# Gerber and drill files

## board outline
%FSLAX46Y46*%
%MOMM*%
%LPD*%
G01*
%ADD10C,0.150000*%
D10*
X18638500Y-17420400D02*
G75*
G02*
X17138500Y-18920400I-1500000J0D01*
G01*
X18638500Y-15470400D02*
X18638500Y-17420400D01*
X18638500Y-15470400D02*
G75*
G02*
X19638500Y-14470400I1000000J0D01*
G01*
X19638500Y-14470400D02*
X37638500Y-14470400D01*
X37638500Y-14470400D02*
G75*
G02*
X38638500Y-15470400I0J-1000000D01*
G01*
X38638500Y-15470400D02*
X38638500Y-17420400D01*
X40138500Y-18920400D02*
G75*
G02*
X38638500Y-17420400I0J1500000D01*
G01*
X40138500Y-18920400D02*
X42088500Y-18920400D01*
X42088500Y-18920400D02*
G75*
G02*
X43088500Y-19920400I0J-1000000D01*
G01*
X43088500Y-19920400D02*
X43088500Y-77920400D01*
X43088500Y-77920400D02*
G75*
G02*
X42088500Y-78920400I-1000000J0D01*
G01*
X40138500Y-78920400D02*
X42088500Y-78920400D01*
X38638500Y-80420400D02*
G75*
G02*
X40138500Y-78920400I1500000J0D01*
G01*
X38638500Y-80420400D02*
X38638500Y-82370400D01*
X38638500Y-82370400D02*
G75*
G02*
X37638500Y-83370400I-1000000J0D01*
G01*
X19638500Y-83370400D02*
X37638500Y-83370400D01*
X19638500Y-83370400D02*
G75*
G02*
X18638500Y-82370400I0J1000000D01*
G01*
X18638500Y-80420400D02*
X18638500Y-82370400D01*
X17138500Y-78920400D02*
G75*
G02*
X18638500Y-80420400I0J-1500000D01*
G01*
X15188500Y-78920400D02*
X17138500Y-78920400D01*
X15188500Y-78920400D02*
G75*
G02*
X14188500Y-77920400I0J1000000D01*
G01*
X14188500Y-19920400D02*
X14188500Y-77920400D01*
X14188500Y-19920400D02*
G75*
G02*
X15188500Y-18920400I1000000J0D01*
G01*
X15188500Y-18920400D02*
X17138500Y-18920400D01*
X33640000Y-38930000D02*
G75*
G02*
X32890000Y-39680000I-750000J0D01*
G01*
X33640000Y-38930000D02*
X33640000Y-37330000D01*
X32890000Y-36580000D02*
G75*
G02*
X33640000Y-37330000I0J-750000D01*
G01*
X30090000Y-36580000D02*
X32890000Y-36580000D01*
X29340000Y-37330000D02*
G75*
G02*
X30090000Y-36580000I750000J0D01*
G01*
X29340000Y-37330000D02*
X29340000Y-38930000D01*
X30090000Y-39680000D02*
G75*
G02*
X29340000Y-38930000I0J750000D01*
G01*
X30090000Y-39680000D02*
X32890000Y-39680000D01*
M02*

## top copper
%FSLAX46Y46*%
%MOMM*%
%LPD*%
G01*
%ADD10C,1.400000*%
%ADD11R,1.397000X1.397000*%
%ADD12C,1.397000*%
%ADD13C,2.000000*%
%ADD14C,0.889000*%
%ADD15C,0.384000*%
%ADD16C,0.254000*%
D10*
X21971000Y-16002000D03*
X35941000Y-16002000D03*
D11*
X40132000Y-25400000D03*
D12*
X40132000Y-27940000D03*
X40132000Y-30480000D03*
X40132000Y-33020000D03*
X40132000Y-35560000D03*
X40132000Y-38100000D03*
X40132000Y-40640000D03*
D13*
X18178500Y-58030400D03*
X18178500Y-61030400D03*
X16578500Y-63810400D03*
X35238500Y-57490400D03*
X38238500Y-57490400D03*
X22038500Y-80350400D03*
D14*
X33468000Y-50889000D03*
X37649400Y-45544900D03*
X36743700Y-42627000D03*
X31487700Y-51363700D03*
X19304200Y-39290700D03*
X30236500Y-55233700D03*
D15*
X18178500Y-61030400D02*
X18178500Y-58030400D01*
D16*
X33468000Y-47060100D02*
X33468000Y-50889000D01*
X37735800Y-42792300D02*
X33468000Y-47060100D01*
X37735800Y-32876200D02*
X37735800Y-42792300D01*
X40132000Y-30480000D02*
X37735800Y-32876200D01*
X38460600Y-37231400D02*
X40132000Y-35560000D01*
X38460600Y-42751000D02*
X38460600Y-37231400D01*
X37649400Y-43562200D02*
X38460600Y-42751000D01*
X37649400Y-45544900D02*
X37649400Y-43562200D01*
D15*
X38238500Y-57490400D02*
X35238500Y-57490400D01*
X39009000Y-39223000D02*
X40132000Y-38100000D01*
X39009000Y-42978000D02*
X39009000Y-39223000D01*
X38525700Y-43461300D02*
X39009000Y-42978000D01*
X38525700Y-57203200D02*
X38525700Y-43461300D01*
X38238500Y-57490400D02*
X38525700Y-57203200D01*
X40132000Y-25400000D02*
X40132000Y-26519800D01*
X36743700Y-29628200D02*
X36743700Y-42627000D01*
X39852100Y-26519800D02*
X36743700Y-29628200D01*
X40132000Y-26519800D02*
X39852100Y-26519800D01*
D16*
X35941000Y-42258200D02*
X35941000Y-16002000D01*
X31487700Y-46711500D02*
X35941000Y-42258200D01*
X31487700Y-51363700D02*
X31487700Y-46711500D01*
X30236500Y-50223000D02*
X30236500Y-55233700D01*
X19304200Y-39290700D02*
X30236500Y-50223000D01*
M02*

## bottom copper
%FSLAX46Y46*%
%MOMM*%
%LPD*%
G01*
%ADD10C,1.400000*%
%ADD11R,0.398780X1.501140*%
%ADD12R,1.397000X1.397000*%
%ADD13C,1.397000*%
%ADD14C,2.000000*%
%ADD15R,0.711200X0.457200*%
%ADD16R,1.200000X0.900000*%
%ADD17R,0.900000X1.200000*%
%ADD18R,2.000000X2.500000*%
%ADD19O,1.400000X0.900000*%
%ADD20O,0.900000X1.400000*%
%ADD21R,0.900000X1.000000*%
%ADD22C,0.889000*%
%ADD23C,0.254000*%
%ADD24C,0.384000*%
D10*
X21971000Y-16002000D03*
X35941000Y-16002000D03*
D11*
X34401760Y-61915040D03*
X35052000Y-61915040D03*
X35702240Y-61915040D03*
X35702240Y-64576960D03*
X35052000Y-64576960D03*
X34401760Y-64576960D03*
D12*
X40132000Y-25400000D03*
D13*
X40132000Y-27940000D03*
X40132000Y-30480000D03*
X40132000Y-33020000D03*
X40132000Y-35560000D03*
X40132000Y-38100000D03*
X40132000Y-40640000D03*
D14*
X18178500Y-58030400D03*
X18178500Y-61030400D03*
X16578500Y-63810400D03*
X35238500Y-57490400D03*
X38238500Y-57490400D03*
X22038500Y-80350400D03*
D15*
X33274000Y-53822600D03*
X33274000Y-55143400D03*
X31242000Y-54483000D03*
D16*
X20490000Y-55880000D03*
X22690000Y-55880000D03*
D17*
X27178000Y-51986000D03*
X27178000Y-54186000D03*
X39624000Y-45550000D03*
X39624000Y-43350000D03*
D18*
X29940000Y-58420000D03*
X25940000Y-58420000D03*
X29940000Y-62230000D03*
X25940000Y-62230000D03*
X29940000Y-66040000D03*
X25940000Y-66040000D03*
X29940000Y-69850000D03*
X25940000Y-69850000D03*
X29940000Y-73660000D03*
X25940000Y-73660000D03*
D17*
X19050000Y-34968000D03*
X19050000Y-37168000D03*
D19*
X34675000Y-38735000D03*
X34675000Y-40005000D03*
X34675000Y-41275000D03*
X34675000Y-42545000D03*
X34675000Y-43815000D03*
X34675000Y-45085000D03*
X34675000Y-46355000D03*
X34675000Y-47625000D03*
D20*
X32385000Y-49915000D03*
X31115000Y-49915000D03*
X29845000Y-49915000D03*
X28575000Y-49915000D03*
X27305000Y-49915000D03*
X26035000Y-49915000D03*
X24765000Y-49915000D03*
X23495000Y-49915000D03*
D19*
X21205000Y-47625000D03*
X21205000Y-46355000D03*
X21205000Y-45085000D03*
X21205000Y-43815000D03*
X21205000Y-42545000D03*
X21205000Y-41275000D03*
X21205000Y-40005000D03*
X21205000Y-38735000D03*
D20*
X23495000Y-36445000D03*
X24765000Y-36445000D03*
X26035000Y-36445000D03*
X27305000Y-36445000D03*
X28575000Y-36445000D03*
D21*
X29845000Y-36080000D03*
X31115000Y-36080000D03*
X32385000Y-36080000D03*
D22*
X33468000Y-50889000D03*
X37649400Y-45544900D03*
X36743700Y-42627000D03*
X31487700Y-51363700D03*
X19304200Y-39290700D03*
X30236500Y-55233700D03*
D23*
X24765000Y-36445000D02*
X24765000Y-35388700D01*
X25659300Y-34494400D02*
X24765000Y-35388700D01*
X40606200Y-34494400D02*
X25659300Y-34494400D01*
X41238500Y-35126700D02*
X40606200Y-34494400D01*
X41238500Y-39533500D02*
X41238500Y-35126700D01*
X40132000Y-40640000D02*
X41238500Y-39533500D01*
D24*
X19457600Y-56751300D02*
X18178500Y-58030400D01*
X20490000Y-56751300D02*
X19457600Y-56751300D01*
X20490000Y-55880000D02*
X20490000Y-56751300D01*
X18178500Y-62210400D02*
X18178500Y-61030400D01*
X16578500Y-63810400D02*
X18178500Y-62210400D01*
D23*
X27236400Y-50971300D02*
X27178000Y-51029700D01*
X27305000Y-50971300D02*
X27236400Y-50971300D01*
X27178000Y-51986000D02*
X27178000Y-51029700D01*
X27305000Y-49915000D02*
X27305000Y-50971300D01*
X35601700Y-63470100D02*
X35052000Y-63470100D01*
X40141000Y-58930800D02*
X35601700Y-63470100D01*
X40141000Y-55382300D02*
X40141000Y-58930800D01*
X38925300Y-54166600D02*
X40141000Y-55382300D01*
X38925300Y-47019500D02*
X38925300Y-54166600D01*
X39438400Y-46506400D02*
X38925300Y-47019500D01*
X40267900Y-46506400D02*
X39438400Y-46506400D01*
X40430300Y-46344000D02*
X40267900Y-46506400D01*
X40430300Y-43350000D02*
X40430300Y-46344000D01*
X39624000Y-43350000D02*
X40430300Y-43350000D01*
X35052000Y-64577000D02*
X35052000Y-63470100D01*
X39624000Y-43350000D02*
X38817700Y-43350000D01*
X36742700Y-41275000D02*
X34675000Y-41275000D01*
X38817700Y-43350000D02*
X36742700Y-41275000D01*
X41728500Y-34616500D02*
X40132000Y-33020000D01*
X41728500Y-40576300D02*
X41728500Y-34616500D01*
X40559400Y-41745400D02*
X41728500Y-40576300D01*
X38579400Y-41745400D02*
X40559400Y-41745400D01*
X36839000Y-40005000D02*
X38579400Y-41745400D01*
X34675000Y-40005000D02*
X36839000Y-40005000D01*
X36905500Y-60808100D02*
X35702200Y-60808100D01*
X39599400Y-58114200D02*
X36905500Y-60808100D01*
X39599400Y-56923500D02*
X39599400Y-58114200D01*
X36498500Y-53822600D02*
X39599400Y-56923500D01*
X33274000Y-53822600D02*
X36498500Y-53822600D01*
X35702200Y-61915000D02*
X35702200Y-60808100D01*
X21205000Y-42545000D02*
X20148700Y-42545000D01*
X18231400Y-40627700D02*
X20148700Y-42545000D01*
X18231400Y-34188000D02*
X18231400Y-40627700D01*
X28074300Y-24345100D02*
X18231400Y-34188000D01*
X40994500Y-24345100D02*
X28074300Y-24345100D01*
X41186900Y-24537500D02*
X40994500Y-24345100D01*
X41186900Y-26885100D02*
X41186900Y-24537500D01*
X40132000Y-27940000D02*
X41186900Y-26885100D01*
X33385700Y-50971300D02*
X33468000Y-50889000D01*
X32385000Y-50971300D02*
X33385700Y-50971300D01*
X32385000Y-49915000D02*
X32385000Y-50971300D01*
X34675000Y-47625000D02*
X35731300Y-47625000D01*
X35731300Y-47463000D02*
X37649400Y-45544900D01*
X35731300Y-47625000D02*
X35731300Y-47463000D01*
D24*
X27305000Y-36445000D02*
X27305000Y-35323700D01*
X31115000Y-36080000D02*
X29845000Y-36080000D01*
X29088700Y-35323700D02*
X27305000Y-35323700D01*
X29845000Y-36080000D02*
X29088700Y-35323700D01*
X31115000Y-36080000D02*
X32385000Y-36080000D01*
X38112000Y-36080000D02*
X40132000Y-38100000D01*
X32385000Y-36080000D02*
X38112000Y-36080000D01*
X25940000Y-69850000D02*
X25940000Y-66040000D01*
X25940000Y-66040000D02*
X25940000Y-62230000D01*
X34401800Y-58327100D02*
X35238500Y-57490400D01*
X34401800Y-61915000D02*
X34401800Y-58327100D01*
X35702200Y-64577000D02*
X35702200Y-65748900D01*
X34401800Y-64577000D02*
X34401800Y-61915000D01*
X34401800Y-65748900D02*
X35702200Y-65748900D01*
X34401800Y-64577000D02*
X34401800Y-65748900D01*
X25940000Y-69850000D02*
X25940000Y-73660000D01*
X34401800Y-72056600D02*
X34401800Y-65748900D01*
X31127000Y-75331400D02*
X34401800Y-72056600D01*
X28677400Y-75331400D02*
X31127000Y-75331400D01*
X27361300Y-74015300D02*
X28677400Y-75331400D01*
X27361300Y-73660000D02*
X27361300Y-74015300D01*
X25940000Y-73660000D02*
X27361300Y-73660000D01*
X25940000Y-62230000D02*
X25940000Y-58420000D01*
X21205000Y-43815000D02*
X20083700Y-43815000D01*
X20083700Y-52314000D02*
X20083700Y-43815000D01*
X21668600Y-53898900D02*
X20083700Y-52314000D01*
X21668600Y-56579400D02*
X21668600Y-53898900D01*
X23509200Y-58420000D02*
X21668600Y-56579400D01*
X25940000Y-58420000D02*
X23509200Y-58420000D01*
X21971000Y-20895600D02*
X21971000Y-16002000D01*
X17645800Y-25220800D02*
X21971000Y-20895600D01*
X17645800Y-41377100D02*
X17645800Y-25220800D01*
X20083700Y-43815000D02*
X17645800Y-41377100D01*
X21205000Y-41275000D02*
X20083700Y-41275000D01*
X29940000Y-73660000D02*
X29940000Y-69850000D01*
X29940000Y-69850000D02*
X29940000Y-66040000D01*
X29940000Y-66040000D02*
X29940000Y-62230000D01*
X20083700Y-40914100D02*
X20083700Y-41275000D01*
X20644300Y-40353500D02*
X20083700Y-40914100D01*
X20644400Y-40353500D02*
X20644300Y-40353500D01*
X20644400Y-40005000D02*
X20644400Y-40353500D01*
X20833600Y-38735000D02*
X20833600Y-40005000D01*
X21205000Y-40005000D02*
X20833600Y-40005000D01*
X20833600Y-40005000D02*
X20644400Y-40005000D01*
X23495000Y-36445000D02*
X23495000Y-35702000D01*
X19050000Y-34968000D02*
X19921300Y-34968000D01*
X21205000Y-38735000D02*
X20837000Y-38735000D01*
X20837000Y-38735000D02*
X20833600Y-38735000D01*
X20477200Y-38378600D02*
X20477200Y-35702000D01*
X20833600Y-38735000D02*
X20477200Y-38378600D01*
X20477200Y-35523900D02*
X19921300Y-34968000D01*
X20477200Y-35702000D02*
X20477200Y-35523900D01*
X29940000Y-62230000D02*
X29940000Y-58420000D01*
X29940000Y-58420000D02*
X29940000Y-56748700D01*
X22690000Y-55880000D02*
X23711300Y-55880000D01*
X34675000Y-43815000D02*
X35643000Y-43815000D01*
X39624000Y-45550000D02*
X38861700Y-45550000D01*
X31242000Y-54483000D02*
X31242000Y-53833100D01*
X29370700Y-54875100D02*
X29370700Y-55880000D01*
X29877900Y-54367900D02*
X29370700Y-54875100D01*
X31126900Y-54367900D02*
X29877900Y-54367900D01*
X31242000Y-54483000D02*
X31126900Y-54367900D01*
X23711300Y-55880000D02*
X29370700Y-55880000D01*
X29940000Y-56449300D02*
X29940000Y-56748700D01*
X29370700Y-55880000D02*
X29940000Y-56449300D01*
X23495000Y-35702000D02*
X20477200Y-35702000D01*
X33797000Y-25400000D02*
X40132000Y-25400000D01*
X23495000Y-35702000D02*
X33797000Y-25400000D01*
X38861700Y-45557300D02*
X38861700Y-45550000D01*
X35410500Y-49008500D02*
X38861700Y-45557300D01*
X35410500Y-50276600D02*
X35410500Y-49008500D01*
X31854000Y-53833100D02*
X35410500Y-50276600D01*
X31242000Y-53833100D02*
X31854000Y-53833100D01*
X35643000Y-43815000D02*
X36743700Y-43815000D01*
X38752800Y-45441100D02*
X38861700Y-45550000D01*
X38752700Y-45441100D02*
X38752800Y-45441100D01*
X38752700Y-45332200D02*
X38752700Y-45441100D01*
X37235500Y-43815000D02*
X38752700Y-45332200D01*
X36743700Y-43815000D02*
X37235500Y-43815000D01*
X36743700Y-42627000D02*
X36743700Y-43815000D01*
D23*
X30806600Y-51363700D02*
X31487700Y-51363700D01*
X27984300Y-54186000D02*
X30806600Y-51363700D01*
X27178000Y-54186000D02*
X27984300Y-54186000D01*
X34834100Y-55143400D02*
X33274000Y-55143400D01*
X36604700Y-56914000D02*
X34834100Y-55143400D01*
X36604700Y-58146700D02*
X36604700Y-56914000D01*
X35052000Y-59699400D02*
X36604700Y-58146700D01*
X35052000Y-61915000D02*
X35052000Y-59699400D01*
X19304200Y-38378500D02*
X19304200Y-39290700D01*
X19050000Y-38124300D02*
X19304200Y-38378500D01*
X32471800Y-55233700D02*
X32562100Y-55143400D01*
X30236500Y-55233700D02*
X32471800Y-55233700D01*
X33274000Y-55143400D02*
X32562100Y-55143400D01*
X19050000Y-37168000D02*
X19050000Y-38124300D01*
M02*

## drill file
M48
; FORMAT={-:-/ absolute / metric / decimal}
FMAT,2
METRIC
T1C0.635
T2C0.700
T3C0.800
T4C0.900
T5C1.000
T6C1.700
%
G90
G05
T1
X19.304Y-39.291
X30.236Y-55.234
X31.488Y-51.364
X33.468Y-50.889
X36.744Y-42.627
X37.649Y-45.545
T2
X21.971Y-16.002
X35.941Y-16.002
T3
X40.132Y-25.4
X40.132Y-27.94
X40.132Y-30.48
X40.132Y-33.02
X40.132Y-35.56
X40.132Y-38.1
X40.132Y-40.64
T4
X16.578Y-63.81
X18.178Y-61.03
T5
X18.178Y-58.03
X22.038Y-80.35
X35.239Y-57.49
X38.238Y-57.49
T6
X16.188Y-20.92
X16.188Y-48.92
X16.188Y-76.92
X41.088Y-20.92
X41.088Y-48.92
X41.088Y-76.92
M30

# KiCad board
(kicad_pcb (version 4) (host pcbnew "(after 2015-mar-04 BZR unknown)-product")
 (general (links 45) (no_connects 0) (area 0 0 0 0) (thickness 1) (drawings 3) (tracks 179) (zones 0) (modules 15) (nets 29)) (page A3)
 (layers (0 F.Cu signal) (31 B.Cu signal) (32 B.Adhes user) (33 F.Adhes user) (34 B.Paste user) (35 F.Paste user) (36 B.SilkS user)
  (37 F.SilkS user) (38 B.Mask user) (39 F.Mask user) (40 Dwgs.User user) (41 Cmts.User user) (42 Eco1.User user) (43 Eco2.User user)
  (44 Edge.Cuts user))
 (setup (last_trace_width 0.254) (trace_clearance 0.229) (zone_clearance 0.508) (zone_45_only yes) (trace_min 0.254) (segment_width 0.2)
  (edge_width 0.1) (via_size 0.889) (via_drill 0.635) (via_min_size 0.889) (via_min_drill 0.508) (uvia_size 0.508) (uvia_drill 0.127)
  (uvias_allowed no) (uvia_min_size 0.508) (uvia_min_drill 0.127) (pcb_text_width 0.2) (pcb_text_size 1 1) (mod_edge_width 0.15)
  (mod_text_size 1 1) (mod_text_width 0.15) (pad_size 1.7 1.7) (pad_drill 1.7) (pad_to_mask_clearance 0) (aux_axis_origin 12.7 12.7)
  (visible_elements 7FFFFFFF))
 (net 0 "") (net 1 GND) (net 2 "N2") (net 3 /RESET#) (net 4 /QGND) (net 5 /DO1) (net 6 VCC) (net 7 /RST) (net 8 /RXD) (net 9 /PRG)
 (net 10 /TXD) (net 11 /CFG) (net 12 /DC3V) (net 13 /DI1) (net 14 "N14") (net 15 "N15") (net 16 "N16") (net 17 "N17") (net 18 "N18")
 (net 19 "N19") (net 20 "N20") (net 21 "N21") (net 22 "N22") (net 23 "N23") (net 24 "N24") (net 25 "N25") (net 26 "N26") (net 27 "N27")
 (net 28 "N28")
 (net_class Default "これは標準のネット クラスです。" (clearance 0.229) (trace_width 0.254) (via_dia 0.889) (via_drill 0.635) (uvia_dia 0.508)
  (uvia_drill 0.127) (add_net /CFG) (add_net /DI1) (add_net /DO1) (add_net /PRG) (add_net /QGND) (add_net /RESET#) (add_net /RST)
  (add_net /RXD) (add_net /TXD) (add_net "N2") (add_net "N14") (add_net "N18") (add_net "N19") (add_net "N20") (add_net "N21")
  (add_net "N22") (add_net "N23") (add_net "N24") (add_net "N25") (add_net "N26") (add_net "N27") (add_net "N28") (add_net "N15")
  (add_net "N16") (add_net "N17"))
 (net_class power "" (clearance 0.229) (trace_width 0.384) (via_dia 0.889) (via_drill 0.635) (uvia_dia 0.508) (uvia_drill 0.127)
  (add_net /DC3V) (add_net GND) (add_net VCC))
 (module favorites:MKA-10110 (layer F.Cu) (at 28.956 16.002)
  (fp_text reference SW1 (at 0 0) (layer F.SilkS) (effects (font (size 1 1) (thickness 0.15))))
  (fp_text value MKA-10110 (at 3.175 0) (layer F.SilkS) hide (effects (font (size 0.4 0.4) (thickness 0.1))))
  (pad 1 thru_hole circle (at -6.985 0) (size 1.4 1.4) (drill 0.7) (layers *.Cu *.Mask F.SilkS) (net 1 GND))
  (pad 2 thru_hole circle (at 6.985 0) (size 1.4 1.4) (drill 0.7) (layers *.Cu *.Mask F.SilkS) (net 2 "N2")))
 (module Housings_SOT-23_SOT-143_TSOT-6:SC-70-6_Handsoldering (layer B.Cu) (at 35.052 63.246)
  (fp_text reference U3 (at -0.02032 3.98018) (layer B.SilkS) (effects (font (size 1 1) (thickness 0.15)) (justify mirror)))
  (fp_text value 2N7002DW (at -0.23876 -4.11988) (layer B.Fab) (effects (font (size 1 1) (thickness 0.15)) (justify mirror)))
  (pad 1 smd rect (at -0.65024 -1.33096) (size 0.39878 1.50114) (layers B.Cu B.Paste B.Mask) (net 1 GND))
  (pad 2 smd rect (at 0 -1.33096) (size 0.39878 1.50114) (layers B.Cu B.Paste B.Mask) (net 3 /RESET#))
  (pad 3 smd rect (at 0.65024 -1.33096) (size 0.39878 1.50114) (layers B.Cu B.Paste B.Mask) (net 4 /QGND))
  (pad 4 smd rect (at 0.65024 1.33096) (size 0.39878 1.50114) (layers B.Cu B.Paste B.Mask) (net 1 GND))
  (pad 5 smd rect (at 0 1.33096) (size 0.39878 1.50114) (layers B.Cu B.Paste B.Mask) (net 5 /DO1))
  (pad 6 smd rect (at -0.65024 1.33096) (size 0.39878 1.50114) (layers B.Cu B.Paste B.Mask) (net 1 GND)))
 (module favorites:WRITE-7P (layer F.Cu) (at 40.132 33.02 270)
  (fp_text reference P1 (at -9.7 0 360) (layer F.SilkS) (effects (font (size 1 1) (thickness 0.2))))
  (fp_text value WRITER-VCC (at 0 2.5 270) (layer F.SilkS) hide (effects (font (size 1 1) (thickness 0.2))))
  (pad 0 thru_hole rect (at -7.62 0 270) (size 1.397 1.397) (drill 0.8) (layers *.Cu *.Mask F.SilkS) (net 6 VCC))
  (pad 1 thru_hole circle (at -5.08 0 270) (size 1.397 1.397) (drill 0.8) (layers *.Cu *.SilkS *.Mask) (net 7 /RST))
  (pad 2 thru_hole circle (at -2.54 0 270) (size 1.397 1.397) (drill 0.8) (layers *.Cu *.SilkS *.Mask) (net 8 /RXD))
  (pad 3 thru_hole circle (at 0 0 270) (size 1.397 1.397) (drill 0.8) (layers *.Cu *.SilkS *.Mask) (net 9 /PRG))
  (pad 4 thru_hole circle (at 2.54 0 270) (size 1.397 1.397) (drill 0.8) (layers *.Cu *.SilkS *.Mask) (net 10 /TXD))
  (pad 5 thru_hole circle (at 5.08 0 270) (size 1.397 1.397) (drill 0.8) (layers *.Cu *.SilkS *.Mask) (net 1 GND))
  (pad 6 thru_hole circle (at 7.62 0 270) (size 1.397 1.397) (drill 0.8) (layers *.Cu *.SilkS *.Mask) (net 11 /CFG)))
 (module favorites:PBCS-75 (layer F.Cu) (at 28.6385 48.9204)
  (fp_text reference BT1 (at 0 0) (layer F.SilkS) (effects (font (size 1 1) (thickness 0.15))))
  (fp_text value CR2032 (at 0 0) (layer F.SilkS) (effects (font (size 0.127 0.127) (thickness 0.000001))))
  (fp_arc (start -11.5 -31.5) (end -10 -31.5) (angle 90) (layer Edge.Cuts) (width 0.15))
  (fp_line (start -10 -33.45) (end -10 -31.5) (layer Edge.Cuts) (width 0.15))
  (fp_arc (start -9 -33.45) (end -10 -33.45) (angle 90) (layer Edge.Cuts) (width 0.15))
  (fp_line (start -9 -34.45) (end 9 -34.45) (layer Edge.Cuts) (width 0.15))
  (fp_arc (start 9 -33.45) (end 9 -34.45) (angle 90) (layer Edge.Cuts) (width 0.15))
  (fp_line (start 10 -33.45) (end 10 -31.5) (layer Edge.Cuts) (width 0.15))
  (fp_arc (start 11.5 -31.5) (end 11.5 -30) (angle 90) (layer Edge.Cuts) (width 0.15))
  (fp_line (start 11.5 -30) (end 13.45 -30) (layer Edge.Cuts) (width 0.15))
  (fp_arc (start 13.45 -29) (end 13.45 -30) (angle 90) (layer Edge.Cuts) (width 0.15))
  (fp_line (start 14.45 -29) (end 14.45 29) (layer Edge.Cuts) (width 0.15))
  (fp_arc (start 13.45 29) (end 14.45 29) (angle 90) (layer Edge.Cuts) (width 0.15))
  (fp_line (start 11.5 30) (end 13.45 30) (layer Edge.Cuts) (width 0.15))
  (fp_arc (start 11.5 31.5) (end 10 31.5) (angle 90) (layer Edge.Cuts) (width 0.15))
  (fp_line (start 10 31.5) (end 10 33.45) (layer Edge.Cuts) (width 0.15))
  (fp_arc (start 9 33.45) (end 10 33.45) (angle 90) (layer Edge.Cuts) (width 0.15))
  (fp_line (start -9 34.45) (end 9 34.45) (layer Edge.Cuts) (width 0.15))
  (fp_arc (start -9 33.45) (end -9 34.45) (angle 90) (layer Edge.Cuts) (width 0.15))
  (fp_line (start -10 31.5) (end -10 33.45) (layer Edge.Cuts) (width 0.15))
  (fp_arc (start -11.5 31.5) (end -11.5 30) (angle 90) (layer Edge.Cuts) (width 0.15))
  (fp_line (start -13.45 30) (end -11.5 30) (layer Edge.Cuts) (width 0.15))
  (fp_arc (start -13.45 29) (end -13.45 30) (angle 90) (layer Edge.Cuts) (width 0.15))
  (fp_line (start -14.45 -29) (end -14.45 29) (layer Edge.Cuts) (width 0.15))
  (fp_arc (start -13.45 -29) (end -14.45 -29) (angle 90) (layer Edge.Cuts) (width 0.15))
  (fp_line (start -13.45 -30) (end -11.5 -30) (layer Edge.Cuts) (width 0.15))
  (pad 1 thru_hole circle (at -10.46 9.11) (size 2 2) (drill 1) (layers *.Cu *.Mask F.SilkS) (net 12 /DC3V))
  (pad 1 thru_hole circle (at -10.46 12.11) (size 2 2) (drill 0.9) (layers *.Cu *.Mask F.SilkS) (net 12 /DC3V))
  (pad 1 thru_hole circle (at -12.06 14.89) (size 2 2) (drill 0.9) (layers *.Cu *.Mask F.SilkS) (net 12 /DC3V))
  (pad 2 thru_hole circle (at 6.6 8.57) (size 2 2) (drill 1) (layers *.Cu *.Mask F.SilkS) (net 1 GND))
  (pad 2 thru_hole circle (at 9.6 8.57) (size 2 2) (drill 1) (layers *.Cu *.Mask F.SilkS) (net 1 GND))
  (pad "" thru_hole circle (at -6.6 31.43) (size 2 2) (drill 1) (layers *.Cu *.Mask F.SilkS))
  (pad "" np_thru_hole circle (at 12.45 28) (size 1.7 1.7) (drill 1.7) (layers *.Cu *.Mask F.SilkS) (clearance 1))
  (pad "" np_thru_hole circle (at -12.45 28) (size 1.7 1.7) (drill 1.7) (layers *.Cu *.Mask F.SilkS) (clearance 1))
  (pad "" np_thru_hole circle (at 12.45 0) (size 1.7 1.7) (drill 1.7) (layers *.Cu *.Mask F.SilkS) (clearance 1))
  (pad "" np_thru_hole circle (at -12.45 0) (size 1.7 1.7) (drill 1.7) (layers *.Cu *.Mask F.SilkS) (clearance 1))
  (pad "" np_thru_hole circle (at -12.45 -28) (size 1.7 1.7) (drill 1.7) (layers *.Cu *.Mask F.SilkS) (clearance 1))
  (pad "" np_thru_hole circle (at 12.45 -28) (size 1.7 1.7) (drill 1.7) (layers *.Cu *.Mask F.SilkS) (clearance 1)))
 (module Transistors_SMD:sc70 (layer B.Cu) (at 32.258 54.483 270)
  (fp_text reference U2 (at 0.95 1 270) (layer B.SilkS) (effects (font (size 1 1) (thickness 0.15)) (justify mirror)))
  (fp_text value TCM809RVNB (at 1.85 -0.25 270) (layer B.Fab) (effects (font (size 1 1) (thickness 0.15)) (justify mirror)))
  (pad 1 smd rect (at -0.6604 -1.016 270) (size 0.4572 0.7112) (layers B.Cu B.Paste B.Mask) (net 4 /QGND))
  (pad 2 smd rect (at 0.6604 -1.016 270) (size 0.4572 0.7112) (layers B.Cu B.Paste B.Mask) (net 3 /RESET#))
  (pad 3 smd rect (at 0 1.016 270) (size 0.4572 0.7112) (layers B.Cu B.Paste B.Mask) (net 6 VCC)))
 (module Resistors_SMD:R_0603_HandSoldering (layer B.Cu) (at 21.59 55.88)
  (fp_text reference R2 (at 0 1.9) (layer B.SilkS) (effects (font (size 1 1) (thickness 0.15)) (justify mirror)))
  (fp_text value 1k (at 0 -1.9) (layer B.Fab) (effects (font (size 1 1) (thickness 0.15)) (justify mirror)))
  (pad 1 smd rect (at -1.1 0) (size 1.2 0.9) (layers B.Cu B.Paste B.Mask) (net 12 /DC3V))
  (pad 2 smd rect (at 1.1 0) (size 1.2 0.9) (layers B.Cu B.Paste B.Mask) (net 6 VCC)))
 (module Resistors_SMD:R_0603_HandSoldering (layer B.Cu) (at 27.178 53.086 270)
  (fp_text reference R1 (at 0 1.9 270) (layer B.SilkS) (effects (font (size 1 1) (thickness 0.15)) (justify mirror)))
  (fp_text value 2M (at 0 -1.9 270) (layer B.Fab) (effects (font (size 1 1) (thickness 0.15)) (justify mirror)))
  (pad 1 smd rect (at -1.1 0 270) (size 1.2 0.9) (layers B.Cu B.Paste B.Mask) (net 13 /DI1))
  (pad 2 smd rect (at 1.1 0 270) (size 1.2 0.9) (layers B.Cu B.Paste B.Mask) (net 2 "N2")))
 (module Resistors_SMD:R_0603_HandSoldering (layer B.Cu) (at 39.624 44.45 90)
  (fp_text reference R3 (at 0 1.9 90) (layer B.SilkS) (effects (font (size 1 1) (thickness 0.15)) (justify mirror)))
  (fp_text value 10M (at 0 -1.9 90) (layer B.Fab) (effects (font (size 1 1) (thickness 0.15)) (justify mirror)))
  (pad 1 smd rect (at -1.1 0 90) (size 1.2 0.9) (layers B.Cu B.Paste B.Mask) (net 6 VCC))
  (pad 2 smd rect (at 1.1 0 90) (size 1.2 0.9) (layers B.Cu B.Paste B.Mask) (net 5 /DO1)))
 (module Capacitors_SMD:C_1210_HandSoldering (layer B.Cu) (at 27.94 58.42 180)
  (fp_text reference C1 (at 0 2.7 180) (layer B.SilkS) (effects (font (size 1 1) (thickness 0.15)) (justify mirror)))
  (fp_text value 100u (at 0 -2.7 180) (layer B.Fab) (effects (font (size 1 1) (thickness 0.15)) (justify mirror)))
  (pad 1 smd rect (at -2 0 180) (size 2 2.5) (layers B.Cu B.Paste B.Mask) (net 6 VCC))
  (pad 2 smd rect (at 2 0 180) (size 2 2.5) (layers B.Cu B.Paste B.Mask) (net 1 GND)))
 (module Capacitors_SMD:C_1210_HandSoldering (layer B.Cu) (at 27.94 62.23 180)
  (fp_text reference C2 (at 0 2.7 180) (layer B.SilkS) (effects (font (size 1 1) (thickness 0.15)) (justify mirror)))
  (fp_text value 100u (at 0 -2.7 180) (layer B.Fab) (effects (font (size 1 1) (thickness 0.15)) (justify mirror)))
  (pad 1 smd rect (at -2 0 180) (size 2 2.5) (layers B.Cu B.Paste B.Mask) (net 6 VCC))
  (pad 2 smd rect (at 2 0 180) (size 2 2.5) (layers B.Cu B.Paste B.Mask) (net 1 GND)))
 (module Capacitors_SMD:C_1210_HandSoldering (layer B.Cu) (at 27.94 66.04 180)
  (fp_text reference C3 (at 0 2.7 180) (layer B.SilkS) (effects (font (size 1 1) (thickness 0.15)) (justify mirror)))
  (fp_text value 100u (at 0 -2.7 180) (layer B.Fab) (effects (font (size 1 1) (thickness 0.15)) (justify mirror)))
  (pad 1 smd rect (at -2 0 180) (size 2 2.5) (layers B.Cu B.Paste B.Mask) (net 6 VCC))
  (pad 2 smd rect (at 2 0 180) (size 2 2.5) (layers B.Cu B.Paste B.Mask) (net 1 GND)))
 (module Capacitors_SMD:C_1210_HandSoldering (layer B.Cu) (at 27.94 69.85 180)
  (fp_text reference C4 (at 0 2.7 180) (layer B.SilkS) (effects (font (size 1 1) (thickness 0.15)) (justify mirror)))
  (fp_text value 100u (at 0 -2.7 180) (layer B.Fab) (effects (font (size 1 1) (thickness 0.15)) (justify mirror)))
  (pad 1 smd rect (at -2 0 180) (size 2 2.5) (layers B.Cu B.Paste B.Mask) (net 6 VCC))
  (pad 2 smd rect (at 2 0 180) (size 2 2.5) (layers B.Cu B.Paste B.Mask) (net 1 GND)))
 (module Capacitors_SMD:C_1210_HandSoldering (layer B.Cu) (at 27.94 73.66 180)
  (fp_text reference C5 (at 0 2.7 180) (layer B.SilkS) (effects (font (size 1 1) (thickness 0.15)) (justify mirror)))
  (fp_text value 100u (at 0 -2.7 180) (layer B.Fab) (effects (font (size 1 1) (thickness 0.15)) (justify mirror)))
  (pad 1 smd rect (at -2 0 180) (size 2 2.5) (layers B.Cu B.Paste B.Mask) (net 6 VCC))
  (pad 2 smd rect (at 2 0 180) (size 2 2.5) (layers B.Cu B.Paste B.Mask) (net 1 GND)))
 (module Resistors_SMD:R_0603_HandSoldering (layer B.Cu) (at 19.05 36.068 270)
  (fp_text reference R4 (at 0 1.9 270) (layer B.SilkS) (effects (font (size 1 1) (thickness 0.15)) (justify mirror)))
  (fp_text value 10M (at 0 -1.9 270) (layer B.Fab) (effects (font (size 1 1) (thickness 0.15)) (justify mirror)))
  (pad 1 smd rect (at -1.1 0 270) (size 1.2 0.9) (layers B.Cu B.Paste B.Mask) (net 6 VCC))
  (pad 2 smd rect (at 1.1 0 270) (size 1.2 0.9) (layers B.Cu B.Paste B.Mask) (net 3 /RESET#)))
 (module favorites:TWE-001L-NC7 (layer B.Cu) (at 27.94 43.18 180)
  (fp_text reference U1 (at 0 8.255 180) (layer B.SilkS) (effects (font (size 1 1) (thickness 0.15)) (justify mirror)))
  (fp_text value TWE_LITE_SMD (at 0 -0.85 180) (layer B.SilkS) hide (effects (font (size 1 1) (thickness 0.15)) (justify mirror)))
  (fp_arc (start -4.95 4.25) (end -4.95 3.5) (angle -90) (layer Edge.Cuts) (width 0.15))
  (fp_line (start -5.7 4.25) (end -5.7 5.85) (layer Edge.Cuts) (width 0.15))
  (fp_arc (start -4.95 5.85) (end -5.7 5.85) (angle -90) (layer Edge.Cuts) (width 0.15))
  (fp_line (start -2.15 6.6) (end -4.95 6.6) (layer Edge.Cuts) (width 0.15))
  (fp_arc (start -2.15 5.85) (end -2.15 6.6) (angle -90) (layer Edge.Cuts) (width 0.15))
  (fp_line (start -1.4 5.85) (end -1.4 4.25) (layer Edge.Cuts) (width 0.15))
  (fp_arc (start -2.15 4.25) (end -1.4 4.25) (angle -90) (layer Edge.Cuts) (width 0.15))
  (fp_line (start -2.15 3.5) (end -4.95 3.5) (layer Edge.Cuts) (width 0.15))
  (pad 1 smd oval (at -6.735 4.445 90) (size 0.9 1.4) (layers B.Cu B.Paste B.Mask) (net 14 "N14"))
  (pad 2 smd oval (at -6.735 3.175 90) (size 0.9 1.4) (layers B.Cu B.Paste B.Mask) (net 9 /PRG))
  (pad 3 smd oval (at -6.735 1.905 90) (size 0.9 1.4) (layers B.Cu B.Paste B.Mask) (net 5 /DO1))
  (pad 4 smd oval (at -6.735 0.635 90) (size 0.9 1.4) (layers B.Cu B.Paste B.Mask) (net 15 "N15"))
  (pad 5 smd oval (at -6.735 -0.635 90) (size 0.9 1.4) (layers B.Cu B.Paste B.Mask) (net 6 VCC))
  (pad 6 smd oval (at -6.735 -1.905 90) (size 0.9 1.4) (layers B.Cu B.Paste B.Mask) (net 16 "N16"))
  (pad 7 smd oval (at -6.735 -3.175 90) (size 0.9 1.4) (layers B.Cu B.Paste B.Mask) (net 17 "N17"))
  (pad 8 smd oval (at -6.735 -4.445 90) (size 0.9 1.4) (layers B.Cu B.Paste B.Mask) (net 10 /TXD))
  (pad 9 smd oval (at -4.445 -6.735 180) (size 0.9 1.4) (layers B.Cu B.Paste B.Mask) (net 8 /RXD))
  (pad 10 smd oval (at -3.175 -6.735 180) (size 0.9 1.4) (layers B.Cu B.Paste B.Mask) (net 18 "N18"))
  (pad 11 smd oval (at -1.905 -6.735 180) (size 0.9 1.4) (layers B.Cu B.Paste B.Mask) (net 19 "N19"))
  (pad 12 smd oval (at -0.635 -6.735 180) (size 0.9 1.4) (layers B.Cu B.Paste B.Mask) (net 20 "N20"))
  (pad 13 smd oval (at 0.635 -6.735 180) (size 0.9 1.4) (layers B.Cu B.Paste B.Mask) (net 13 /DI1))
  (pad 14 smd oval (at 1.905 -6.735 180) (size 0.9 1.4) (layers B.Cu B.Paste B.Mask) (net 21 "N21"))
  (pad 15 smd oval (at 3.175 -6.735 180) (size 0.9 1.4) (layers B.Cu B.Paste B.Mask) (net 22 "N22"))
  (pad 16 smd oval (at 4.445 -6.735 180) (size 0.9 1.4) (layers B.Cu B.Paste B.Mask) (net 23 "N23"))
  (pad 17 smd oval (at 6.735 -4.445 90) (size 0.9 1.4) (layers B.Cu B.Paste B.Mask) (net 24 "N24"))
  (pad 18 smd oval (at 6.735 -3.175 90) (size 0.9 1.4) (layers B.Cu B.Paste B.Mask) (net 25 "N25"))
  (pad 19 smd oval (at 6.735 -1.905 90) (size 0.9 1.4) (layers B.Cu B.Paste B.Mask) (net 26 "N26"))
  (pad 20 smd oval (at 6.735 -0.635 90) (size 0.9 1.4) (layers B.Cu B.Paste B.Mask) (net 1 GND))
  (pad 21 smd oval (at 6.735 0.635 90) (size 0.9 1.4) (layers B.Cu B.Paste B.Mask) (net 7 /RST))
  (pad 22 smd oval (at 6.735 1.905 90) (size 0.9 1.4) (layers B.Cu B.Paste B.Mask) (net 6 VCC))
  (pad 23 smd oval (at 6.735 3.175 90) (size 0.9 1.4) (layers B.Cu B.Paste B.Mask) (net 6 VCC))
  (pad 24 smd oval (at 6.735 4.445 90) (size 0.9 1.4) (layers B.Cu B.Paste B.Mask) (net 6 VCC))
  (pad 25 smd oval (at 4.445 6.735 180) (size 0.9 1.4) (layers B.Cu B.Paste B.Mask) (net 6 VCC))
  (pad 26 smd oval (at 3.175 6.735 180) (size 0.9 1.4) (layers B.Cu B.Paste B.Mask) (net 11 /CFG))
  (pad 27 smd oval (at 1.905 6.735 180) (size 0.9 1.4) (layers B.Cu B.Paste B.Mask) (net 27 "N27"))
  (pad 28 smd oval (at 0.635 6.735 180) (size 0.9 1.4) (layers B.Cu B.Paste B.Mask) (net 1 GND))
  (pad 29 smd oval (at -0.635 6.735 180) (size 0.9 1.4) (layers B.Cu B.Paste B.Mask) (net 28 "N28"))
  (pad 30 smd rect (at -1.905 7.1 180) (size 0.9 1) (layers B.Cu B.Paste B.Mask) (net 1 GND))
  (pad 31 smd rect (at -3.175 7.1 180) (size 0.9 1) (layers B.Cu B.Paste B.Mask) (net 1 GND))
  (pad 32 smd rect (at -4.445 7.1 180) (size 0.9 1) (layers B.Cu B.Paste B.Mask) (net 1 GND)))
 (segment (start 24.765 36.445) (end 24.765 35.3887) (width 0.254) (layer B.Cu) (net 11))
 (segment (start 25.6593 34.4944) (end 24.765 35.3887) (width 0.254) (layer B.Cu) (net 11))
 (segment (start 40.6062 34.4944) (end 25.6593 34.4944) (width 0.254) (layer B.Cu) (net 11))
 (segment (start 41.2385 35.1267) (end 40.6062 34.4944) (width 0.254) (layer B.Cu) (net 11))
 (segment (start 41.2385 39.5335) (end 41.2385 35.1267) (width 0.254) (layer B.Cu) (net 11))
 (segment (start 40.132 40.64) (end 41.2385 39.5335) (width 0.254) (layer B.Cu) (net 11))
 (segment (start 19.4576 56.7513) (end 18.1785 58.0304) (width 0.384) (layer B.Cu) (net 12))
 (segment (start 20.49 56.7513) (end 19.4576 56.7513) (width 0.384) (layer B.Cu) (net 12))
 (segment (start 20.49 55.88) (end 20.49 56.7513) (width 0.384) (layer B.Cu) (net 12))
 (segment (start 18.1785 62.2104) (end 18.1785 61.0304) (width 0.384) (layer B.Cu) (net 12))
 (segment (start 16.5785 63.8104) (end 18.1785 62.2104) (width 0.384) (layer B.Cu) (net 12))
 (segment (start 18.1785 61.0304) (end 18.1785 58.0304) (width 0.384) (layer F.Cu) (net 12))
 (segment (start 27.2364 50.9713) (end 27.178 51.0297) (width 0.254) (layer B.Cu) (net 13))
 (segment (start 27.305 50.9713) (end 27.2364 50.9713) (width 0.254) (layer B.Cu) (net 13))
 (segment (start 27.178 51.986) (end 27.178 51.0297) (width 0.254) (layer B.Cu) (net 13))
 (segment (start 27.305 49.915) (end 27.305 50.9713) (width 0.254) (layer B.Cu) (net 13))
 (segment (start 35.6017 63.4701) (end 35.052 63.4701) (width 0.254) (layer B.Cu) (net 5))
 (segment (start 40.141 58.9308) (end 35.6017 63.4701) (width 0.254) (layer B.Cu) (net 5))
 (segment (start 40.141 55.3823) (end 40.141 58.9308) (width 0.254) (layer B.Cu) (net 5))
 (segment (start 38.9253 54.1666) (end 40.141 55.3823) (width 0.254) (layer B.Cu) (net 5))
 (segment (start 38.9253 47.0195) (end 38.9253 54.1666) (width 0.254) (layer B.Cu) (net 5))
 (segment (start 39.4384 46.5064) (end 38.9253 47.0195) (width 0.254) (layer B.Cu) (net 5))
 (segment (start 40.2679 46.5064) (end 39.4384 46.5064) (width 0.254) (layer B.Cu) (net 5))
 (segment (start 40.4303 46.344) (end 40.2679 46.5064) (width 0.254) (layer B.Cu) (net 5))
 (segment (start 40.4303 43.35) (end 40.4303 46.344) (width 0.254) (layer B.Cu) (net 5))
 (segment (start 39.624 43.35) (end 40.4303 43.35) (width 0.254) (layer B.Cu) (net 5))
 (segment (start 35.052 64.577) (end 35.052 63.4701) (width 0.254) (layer B.Cu) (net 5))
 (segment (start 39.624 43.35) (end 38.8177 43.35) (width 0.254) (layer B.Cu) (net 5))
 (segment (start 36.7427 41.275) (end 34.675 41.275) (width 0.254) (layer B.Cu) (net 5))
 (segment (start 38.8177 43.35) (end 36.7427 41.275) (width 0.254) (layer B.Cu) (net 5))
 (segment (start 41.7285 34.6165) (end 40.132 33.02) (width 0.254) (layer B.Cu) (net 9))
 (segment (start 41.7285 40.5763) (end 41.7285 34.6165) (width 0.254) (layer B.Cu) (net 9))
 (segment (start 40.5594 41.7454) (end 41.7285 40.5763) (width 0.254) (layer B.Cu) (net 9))
 (segment (start 38.5794 41.7454) (end 40.5594 41.7454) (width 0.254) (layer B.Cu) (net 9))
 (segment (start 36.839 40.005) (end 38.5794 41.7454) (width 0.254) (layer B.Cu) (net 9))
 (segment (start 34.675 40.005) (end 36.839 40.005) (width 0.254) (layer B.Cu) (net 9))
 (segment (start 36.9055 60.8081) (end 35.7022 60.8081) (width 0.254) (layer B.Cu) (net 4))
 (segment (start 39.5994 58.1142) (end 36.9055 60.8081) (width 0.254) (layer B.Cu) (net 4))
 (segment (start 39.5994 56.9235) (end 39.5994 58.1142) (width 0.254) (layer B.Cu) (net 4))
 (segment (start 36.4985 53.8226) (end 39.5994 56.9235) (width 0.254) (layer B.Cu) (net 4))
 (segment (start 33.274 53.8226) (end 36.4985 53.8226) (width 0.254) (layer B.Cu) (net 4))
 (segment (start 35.7022 61.915) (end 35.7022 60.8081) (width 0.254) (layer B.Cu) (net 4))
 (segment (start 21.205 42.545) (end 20.1487 42.545) (width 0.254) (layer B.Cu) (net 7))
 (segment (start 18.2314 40.6277) (end 20.1487 42.545) (width 0.254) (layer B.Cu) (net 7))
 (segment (start 18.2314 34.188) (end 18.2314 40.6277) (width 0.254) (layer B.Cu) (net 7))
 (segment (start 28.0743 24.3451) (end 18.2314 34.188) (width 0.254) (layer B.Cu) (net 7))
 (segment (start 40.9945 24.3451) (end 28.0743 24.3451) (width 0.254) (layer B.Cu) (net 7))
 (segment (start 41.1869 24.5375) (end 40.9945 24.3451) (width 0.254) (layer B.Cu) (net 7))
 (segment (start 41.1869 26.8851) (end 41.1869 24.5375) (width 0.254) (layer B.Cu) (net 7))
 (segment (start 40.132 27.94) (end 41.1869 26.8851) (width 0.254) (layer B.Cu) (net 7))
 (via (at 33.468 50.889) (size 0.889) (layers F.Cu B.Cu) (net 8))
 (segment (start 33.3857 50.9713) (end 33.468 50.889) (width 0.254) (layer B.Cu) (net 8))
 (segment (start 32.385 50.9713) (end 33.3857 50.9713) (width 0.254) (layer B.Cu) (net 8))
 (segment (start 33.468 47.0601) (end 33.468 50.889) (width 0.254) (layer F.Cu) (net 8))
 (segment (start 37.7358 42.7923) (end 33.468 47.0601) (width 0.254) (layer F.Cu) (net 8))
 (segment (start 37.7358 32.8762) (end 37.7358 42.7923) (width 0.254) (layer F.Cu) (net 8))
 (segment (start 40.132 30.48) (end 37.7358 32.8762) (width 0.254) (layer F.Cu) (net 8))
 (segment (start 32.385 49.915) (end 32.385 50.9713) (width 0.254) (layer B.Cu) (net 8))
 (via (at 37.6494 45.5449) (size 0.889) (layers F.Cu B.Cu) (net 10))
 (segment (start 34.675 47.625) (end 35.7313 47.625) (width 0.254) (layer B.Cu) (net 10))
 (segment (start 35.7313 47.463) (end 37.6494 45.5449) (width 0.254) (layer B.Cu) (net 10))
 (segment (start 35.7313 47.625) (end 35.7313 47.463) (width 0.254) (layer B.Cu) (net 10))
 (segment (start 38.4606 37.2314) (end 40.132 35.56) (width 0.254) (layer F.Cu) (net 10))
 (segment (start 38.4606 42.751) (end 38.4606 37.2314) (width 0.254) (layer F.Cu) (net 10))
 (segment (start 37.6494 43.5622) (end 38.4606 42.751) (width 0.254) (layer F.Cu) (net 10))
 (segment (start 37.6494 45.5449) (end 37.6494 43.5622) (width 0.254) (layer F.Cu) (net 10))
 (segment (start 27.305 36.445) (end 27.305 35.3237) (width 0.384) (layer B.Cu) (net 1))
 (segment (start 31.115 36.08) (end 29.845 36.08) (width 0.384) (layer B.Cu) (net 1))
 (segment (start 29.0887 35.3237) (end 27.305 35.3237) (width 0.384) (layer B.Cu) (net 1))
 (segment (start 29.845 36.08) (end 29.0887 35.3237) (width 0.384) (layer B.Cu) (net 1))
 (segment (start 31.115 36.08) (end 32.385 36.08) (width 0.384) (layer B.Cu) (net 1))
 (segment (start 38.112 36.08) (end 40.132 38.1) (width 0.384) (layer B.Cu) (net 1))
 (segment (start 32.385 36.08) (end 38.112 36.08) (width 0.384) (layer B.Cu) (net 1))
 (segment (start 25.94 69.85) (end 25.94 66.04) (width 0.384) (layer B.Cu) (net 1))
 (segment (start 25.94 66.04) (end 25.94 62.23) (width 0.384) (layer B.Cu) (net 1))
 (segment (start 34.4018 58.3271) (end 35.2385 57.4904) (width 0.384) (layer B.Cu) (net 1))
 (segment (start 34.4018 61.915) (end 34.4018 58.3271) (width 0.384) (layer B.Cu) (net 1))
 (segment (start 35.7022 64.577) (end 35.7022 65.7489) (width 0.384) (layer B.Cu) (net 1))
 (segment (start 34.4018 64.577) (end 34.4018 61.915) (width 0.384) (layer B.Cu) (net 1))
 (segment (start 34.4018 65.7489) (end 35.7022 65.7489) (width 0.384) (layer B.Cu) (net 1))
 (segment (start 34.4018 64.577) (end 34.4018 65.7489) (width 0.384) (layer B.Cu) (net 1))
 (segment (start 25.94 69.85) (end 25.94 73.66) (width 0.384) (layer B.Cu) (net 1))
 (segment (start 34.4018 72.0566) (end 34.4018 65.7489) (width 0.384) (layer B.Cu) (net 1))
 (segment (start 31.127 75.3314) (end 34.4018 72.0566) (width 0.384) (layer B.Cu) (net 1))
 (segment (start 28.6774 75.3314) (end 31.127 75.3314) (width 0.384) (layer B.Cu) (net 1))
 (segment (start 27.3613 74.0153) (end 28.6774 75.3314) (width 0.384) (layer B.Cu) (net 1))
 (segment (start 27.3613 73.66) (end 27.3613 74.0153) (width 0.384) (layer B.Cu) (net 1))
 (segment (start 25.94 73.66) (end 27.3613 73.66) (width 0.384) (layer B.Cu) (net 1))
 (segment (start 38.2385 57.4904) (end 35.2385 57.4904) (width 0.384) (layer F.Cu) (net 1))
 (segment (start 25.94 62.23) (end 25.94 58.42) (width 0.384) (layer B.Cu) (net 1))
 (segment (start 21.205 43.815) (end 20.0837 43.815) (width 0.384) (layer B.Cu) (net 1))
 (segment (start 20.0837 52.314) (end 20.0837 43.815) (width 0.384) (layer B.Cu) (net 1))
 (segment (start 21.6686 53.8989) (end 20.0837 52.314) (width 0.384) (layer B.Cu) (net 1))
 (segment (start 21.6686 56.5794) (end 21.6686 53.8989) (width 0.384) (layer B.Cu) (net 1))
 (segment (start 23.5092 58.42) (end 21.6686 56.5794) (width 0.384) (layer B.Cu) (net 1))
 (segment (start 25.94 58.42) (end 23.5092 58.42) (width 0.384) (layer B.Cu) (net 1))
 (segment (start 21.971 20.8956) (end 21.971 16.002) (width 0.384) (layer B.Cu) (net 1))
 (segment (start 17.6458 25.2208) (end 21.971 20.8956) (width 0.384) (layer B.Cu) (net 1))
 (segment (start 17.6458 41.3771) (end 17.6458 25.2208) (width 0.384) (layer B.Cu) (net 1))
 (segment (start 20.0837 43.815) (end 17.6458 41.3771) (width 0.384) (layer B.Cu) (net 1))
 (segment (start 39.009 39.223) (end 40.132 38.1) (width 0.384) (layer F.Cu) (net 1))
 (segment (start 39.009 42.978) (end 39.009 39.223) (width 0.384) (layer F.Cu) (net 1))
 (segment (start 38.5257 43.4613) (end 39.009 42.978) (width 0.384) (layer F.Cu) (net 1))
 (segment (start 38.5257 57.2032) (end 38.5257 43.4613) (width 0.384) (layer F.Cu) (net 1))
 (segment (start 38.2385 57.4904) (end 38.5257 57.2032) (width 0.384) (layer F.Cu) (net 1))
 (via (at 36.7437 42.627) (size 0.889) (layers F.Cu B.Cu) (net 6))
 (segment (start 21.205 41.275) (end 20.0837 41.275) (width 0.384) (layer B.Cu) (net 6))
 (segment (start 29.94 73.66) (end 29.94 69.85) (width 0.384) (layer B.Cu) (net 6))
 (segment (start 29.94 69.85) (end 29.94 66.04) (width 0.384) (layer B.Cu) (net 6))
 (segment (start 29.94 66.04) (end 29.94 62.23) (width 0.384) (layer B.Cu) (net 6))
 (segment (start 20.0837 40.9141) (end 20.0837 41.275) (width 0.384) (layer B.Cu) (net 6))
 (segment (start 20.6443 40.3535) (end 20.0837 40.9141) (width 0.384) (layer B.Cu) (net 6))
 (segment (start 20.6444 40.3535) (end 20.6443 40.3535) (width 0.384) (layer B.Cu) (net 6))
 (segment (start 20.6444 40.005) (end 20.6444 40.3535) (width 0.384) (layer B.Cu) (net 6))
 (segment (start 20.8336 38.735) (end 20.8336 40.005) (width 0.384) (layer B.Cu) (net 6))
 (segment (start 21.205 40.005) (end 20.8336 40.005) (width 0.384) (layer B.Cu) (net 6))
 (segment (start 20.8336 40.005) (end 20.6444 40.005) (width 0.384) (layer B.Cu) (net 6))
 (segment (start 23.495 36.445) (end 23.495 35.702) (width 0.384) (layer B.Cu) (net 6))
 (segment (start 19.05 34.968) (end 19.9213 34.968) (width 0.384) (layer B.Cu) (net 6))
 (segment (start 21.205 38.735) (end 20.837 38.735) (width 0.384) (layer B.Cu) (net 6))
 (segment (start 20.837 38.735) (end 20.8336 38.735) (width 0.384) (layer B.Cu) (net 6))
 (segment (start 20.4772 38.3786) (end 20.4772 35.702) (width 0.384) (layer B.Cu) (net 6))
 (segment (start 20.8336 38.735) (end 20.4772 38.3786) (width 0.384) (layer B.Cu) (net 6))
 (segment (start 20.4772 35.5239) (end 19.9213 34.968) (width 0.384) (layer B.Cu) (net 6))
 (segment (start 20.4772 35.702) (end 20.4772 35.5239) (width 0.384) (layer B.Cu) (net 6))
 (segment (start 29.94 62.23) (end 29.94 58.42) (width 0.384) (layer B.Cu) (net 6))
 (segment (start 29.94 58.42) (end 29.94 56.7487) (width 0.384) (layer B.Cu) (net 6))
 (segment (start 22.69 55.88) (end 23.7113 55.88) (width 0.384) (layer B.Cu) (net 6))
 (segment (start 34.675 43.815) (end 35.643 43.815) (width 0.384) (layer B.Cu) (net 6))
 (segment (start 39.624 45.55) (end 38.8617 45.55) (width 0.384) (layer B.Cu) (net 6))
 (segment (start 31.242 54.483) (end 31.242 53.8331) (width 0.384) (layer B.Cu) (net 6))
 (segment (start 29.3707 54.8751) (end 29.3707 55.88) (width 0.384) (layer B.Cu) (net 6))
 (segment (start 29.8779 54.3679) (end 29.3707 54.8751) (width 0.384) (layer B.Cu) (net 6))
 (segment (start 31.1269 54.3679) (end 29.8779 54.3679) (width 0.384) (layer B.Cu) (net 6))
 (segment (start 31.242 54.483) (end 31.1269 54.3679) (width 0.384) (layer B.Cu) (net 6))
 (segment (start 23.7113 55.88) (end 29.3707 55.88) (width 0.384) (layer B.Cu) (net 6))
 (segment (start 29.94 56.4493) (end 29.94 56.7487) (width 0.384) (layer B.Cu) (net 6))
 (segment (start 29.3707 55.88) (end 29.94 56.4493) (width 0.384) (layer B.Cu) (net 6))
 (segment (start 23.495 35.702) (end 20.4772 35.702) (width 0.384) (layer B.Cu) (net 6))
 (segment (start 33.797 25.4) (end 40.132 25.4) (width 0.384) (layer B.Cu) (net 6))
 (segment (start 23.495 35.702) (end 33.797 25.4) (width 0.384) (layer B.Cu) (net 6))
 (segment (start 38.8617 45.5573) (end 38.8617 45.55) (width 0.384) (layer B.Cu) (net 6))
 (segment (start 35.4105 49.0085) (end 38.8617 45.5573) (width 0.384) (layer B.Cu) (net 6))
 (segment (start 35.4105 50.2766) (end 35.4105 49.0085) (width 0.384) (layer B.Cu) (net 6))
 (segment (start 31.854 53.8331) (end 35.4105 50.2766) (width 0.384) (layer B.Cu) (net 6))
 (segment (start 31.242 53.8331) (end 31.854 53.8331) (width 0.384) (layer B.Cu) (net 6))
 (segment (start 40.132 25.4) (end 40.132 26.5198) (width 0.384) (layer F.Cu) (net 6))
 (segment (start 35.643 43.815) (end 36.7437 43.815) (width 0.384) (layer B.Cu) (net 6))
 (segment (start 38.7528 45.4411) (end 38.8617 45.55) (width 0.384) (layer B.Cu) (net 6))
 (segment (start 38.7527 45.4411) (end 38.7528 45.4411) (width 0.384) (layer B.Cu) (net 6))
 (segment (start 38.7527 45.3322) (end 38.7527 45.4411) (width 0.384) (layer B.Cu) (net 6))
 (segment (start 37.2355 43.815) (end 38.7527 45.3322) (width 0.384) (layer B.Cu) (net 6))
 (segment (start 36.7437 43.815) (end 37.2355 43.815) (width 0.384) (layer B.Cu) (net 6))
 (segment (start 36.7437 42.627) (end 36.7437 43.815) (width 0.384) (layer B.Cu) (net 6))
 (segment (start 36.7437 29.6282) (end 36.7437 42.627) (width 0.384) (layer F.Cu) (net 6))
 (segment (start 39.8521 26.5198) (end 36.7437 29.6282) (width 0.384) (layer F.Cu) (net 6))
 (segment (start 40.132 26.5198) (end 39.8521 26.5198) (width 0.384) (layer F.Cu) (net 6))
 (via (at 31.4877 51.3637) (size 0.889) (layers F.Cu B.Cu) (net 2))
 (segment (start 30.8066 51.3637) (end 31.4877 51.3637) (width 0.254) (layer B.Cu) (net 2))
 (segment (start 27.9843 54.186) (end 30.8066 51.3637) (width 0.254) (layer B.Cu) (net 2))
 (segment (start 35.941 42.2582) (end 35.941 16.002) (width 0.254) (layer F.Cu) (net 2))
 (segment (start 31.4877 46.7115) (end 35.941 42.2582) (width 0.254) (layer F.Cu) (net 2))
 (segment (start 31.4877 51.3637) (end 31.4877 46.7115) (width 0.254) (layer F.Cu) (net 2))
 (segment (start 27.178 54.186) (end 27.9843 54.186) (width 0.254) (layer B.Cu) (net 2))
 (via (at 19.3042 39.2907) (size 0.889) (layers F.Cu B.Cu) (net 3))
 (via (at 30.2365 55.2337) (size 0.889) (layers F.Cu B.Cu) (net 3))
 (segment (start 34.8341 55.1434) (end 33.274 55.1434) (width 0.254) (layer B.Cu) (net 3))
 (segment (start 36.6047 56.914) (end 34.8341 55.1434) (width 0.254) (layer B.Cu) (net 3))
 (segment (start 36.6047 58.1467) (end 36.6047 56.914) (width 0.254) (layer B.Cu) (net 3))
 (segment (start 35.052 59.6994) (end 36.6047 58.1467) (width 0.254) (layer B.Cu) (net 3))
 (segment (start 35.052 61.915) (end 35.052 59.6994) (width 0.254) (layer B.Cu) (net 3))
 (segment (start 19.3042 38.3785) (end 19.3042 39.2907) (width 0.254) (layer B.Cu) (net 3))
 (segment (start 19.05 38.1243) (end 19.3042 38.3785) (width 0.254) (layer B.Cu) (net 3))
 (segment (start 30.2365 50.223) (end 30.2365 55.2337) (width 0.254) (layer F.Cu) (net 3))
 (segment (start 19.3042 39.2907) (end 30.2365 50.223) (width 0.254) (layer F.Cu) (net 3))
 (segment (start 32.4718 55.2337) (end 32.5621 55.1434) (width 0.254) (layer B.Cu) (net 3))
 (segment (start 30.2365 55.2337) (end 32.4718 55.2337) (width 0.254) (layer B.Cu) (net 3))
 (segment (start 33.274 55.1434) (end 32.5621 55.1434) (width 0.254) (layer B.Cu) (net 3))
 (segment (start 19.05 37.168) (end 19.05 38.1243) (width 0.254) (layer B.Cu) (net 3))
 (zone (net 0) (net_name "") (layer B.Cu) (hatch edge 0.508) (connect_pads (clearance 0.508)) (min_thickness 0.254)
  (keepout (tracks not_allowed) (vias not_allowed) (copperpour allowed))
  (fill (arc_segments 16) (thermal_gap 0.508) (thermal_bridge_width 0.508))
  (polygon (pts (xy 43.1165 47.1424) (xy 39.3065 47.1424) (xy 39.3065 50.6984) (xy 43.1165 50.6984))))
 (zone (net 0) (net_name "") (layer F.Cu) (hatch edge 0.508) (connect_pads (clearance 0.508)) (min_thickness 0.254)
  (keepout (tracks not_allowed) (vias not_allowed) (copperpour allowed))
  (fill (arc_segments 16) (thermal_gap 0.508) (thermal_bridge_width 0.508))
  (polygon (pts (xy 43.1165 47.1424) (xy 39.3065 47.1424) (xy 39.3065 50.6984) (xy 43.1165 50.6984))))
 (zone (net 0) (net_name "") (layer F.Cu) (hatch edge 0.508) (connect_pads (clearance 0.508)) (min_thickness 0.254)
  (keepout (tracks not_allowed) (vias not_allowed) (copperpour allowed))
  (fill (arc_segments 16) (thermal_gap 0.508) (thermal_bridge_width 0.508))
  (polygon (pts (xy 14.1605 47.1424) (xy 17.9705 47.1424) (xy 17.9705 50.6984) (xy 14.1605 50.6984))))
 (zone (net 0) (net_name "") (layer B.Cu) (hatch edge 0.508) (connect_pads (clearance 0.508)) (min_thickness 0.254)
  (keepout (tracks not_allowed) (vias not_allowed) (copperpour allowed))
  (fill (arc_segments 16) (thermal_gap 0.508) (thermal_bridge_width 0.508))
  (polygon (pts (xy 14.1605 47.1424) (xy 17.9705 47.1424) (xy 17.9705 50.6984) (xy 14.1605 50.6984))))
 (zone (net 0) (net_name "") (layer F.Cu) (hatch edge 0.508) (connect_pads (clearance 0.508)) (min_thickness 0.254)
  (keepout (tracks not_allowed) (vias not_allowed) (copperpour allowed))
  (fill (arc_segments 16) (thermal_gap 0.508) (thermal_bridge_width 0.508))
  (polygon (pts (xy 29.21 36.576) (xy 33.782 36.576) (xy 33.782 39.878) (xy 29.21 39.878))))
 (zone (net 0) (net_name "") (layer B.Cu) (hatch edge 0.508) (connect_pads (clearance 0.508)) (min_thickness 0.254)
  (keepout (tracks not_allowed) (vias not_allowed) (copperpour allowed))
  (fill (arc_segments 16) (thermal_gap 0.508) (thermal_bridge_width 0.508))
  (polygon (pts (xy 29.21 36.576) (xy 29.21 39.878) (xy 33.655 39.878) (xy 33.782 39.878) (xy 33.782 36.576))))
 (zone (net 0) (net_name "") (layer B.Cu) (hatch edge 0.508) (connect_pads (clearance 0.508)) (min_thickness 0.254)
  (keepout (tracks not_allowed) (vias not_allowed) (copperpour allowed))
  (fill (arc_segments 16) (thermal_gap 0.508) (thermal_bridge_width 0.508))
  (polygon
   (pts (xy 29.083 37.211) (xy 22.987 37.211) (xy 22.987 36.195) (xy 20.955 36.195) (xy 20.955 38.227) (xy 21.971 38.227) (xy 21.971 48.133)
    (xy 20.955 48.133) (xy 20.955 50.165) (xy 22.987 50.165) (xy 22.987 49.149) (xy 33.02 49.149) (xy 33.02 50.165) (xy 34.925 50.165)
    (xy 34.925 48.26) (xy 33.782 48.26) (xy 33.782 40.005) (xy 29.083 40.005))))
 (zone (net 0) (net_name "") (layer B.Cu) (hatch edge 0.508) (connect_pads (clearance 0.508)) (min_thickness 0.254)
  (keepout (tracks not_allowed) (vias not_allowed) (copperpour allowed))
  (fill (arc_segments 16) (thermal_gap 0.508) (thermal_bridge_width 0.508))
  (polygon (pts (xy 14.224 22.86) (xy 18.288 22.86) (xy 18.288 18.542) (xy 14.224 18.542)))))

